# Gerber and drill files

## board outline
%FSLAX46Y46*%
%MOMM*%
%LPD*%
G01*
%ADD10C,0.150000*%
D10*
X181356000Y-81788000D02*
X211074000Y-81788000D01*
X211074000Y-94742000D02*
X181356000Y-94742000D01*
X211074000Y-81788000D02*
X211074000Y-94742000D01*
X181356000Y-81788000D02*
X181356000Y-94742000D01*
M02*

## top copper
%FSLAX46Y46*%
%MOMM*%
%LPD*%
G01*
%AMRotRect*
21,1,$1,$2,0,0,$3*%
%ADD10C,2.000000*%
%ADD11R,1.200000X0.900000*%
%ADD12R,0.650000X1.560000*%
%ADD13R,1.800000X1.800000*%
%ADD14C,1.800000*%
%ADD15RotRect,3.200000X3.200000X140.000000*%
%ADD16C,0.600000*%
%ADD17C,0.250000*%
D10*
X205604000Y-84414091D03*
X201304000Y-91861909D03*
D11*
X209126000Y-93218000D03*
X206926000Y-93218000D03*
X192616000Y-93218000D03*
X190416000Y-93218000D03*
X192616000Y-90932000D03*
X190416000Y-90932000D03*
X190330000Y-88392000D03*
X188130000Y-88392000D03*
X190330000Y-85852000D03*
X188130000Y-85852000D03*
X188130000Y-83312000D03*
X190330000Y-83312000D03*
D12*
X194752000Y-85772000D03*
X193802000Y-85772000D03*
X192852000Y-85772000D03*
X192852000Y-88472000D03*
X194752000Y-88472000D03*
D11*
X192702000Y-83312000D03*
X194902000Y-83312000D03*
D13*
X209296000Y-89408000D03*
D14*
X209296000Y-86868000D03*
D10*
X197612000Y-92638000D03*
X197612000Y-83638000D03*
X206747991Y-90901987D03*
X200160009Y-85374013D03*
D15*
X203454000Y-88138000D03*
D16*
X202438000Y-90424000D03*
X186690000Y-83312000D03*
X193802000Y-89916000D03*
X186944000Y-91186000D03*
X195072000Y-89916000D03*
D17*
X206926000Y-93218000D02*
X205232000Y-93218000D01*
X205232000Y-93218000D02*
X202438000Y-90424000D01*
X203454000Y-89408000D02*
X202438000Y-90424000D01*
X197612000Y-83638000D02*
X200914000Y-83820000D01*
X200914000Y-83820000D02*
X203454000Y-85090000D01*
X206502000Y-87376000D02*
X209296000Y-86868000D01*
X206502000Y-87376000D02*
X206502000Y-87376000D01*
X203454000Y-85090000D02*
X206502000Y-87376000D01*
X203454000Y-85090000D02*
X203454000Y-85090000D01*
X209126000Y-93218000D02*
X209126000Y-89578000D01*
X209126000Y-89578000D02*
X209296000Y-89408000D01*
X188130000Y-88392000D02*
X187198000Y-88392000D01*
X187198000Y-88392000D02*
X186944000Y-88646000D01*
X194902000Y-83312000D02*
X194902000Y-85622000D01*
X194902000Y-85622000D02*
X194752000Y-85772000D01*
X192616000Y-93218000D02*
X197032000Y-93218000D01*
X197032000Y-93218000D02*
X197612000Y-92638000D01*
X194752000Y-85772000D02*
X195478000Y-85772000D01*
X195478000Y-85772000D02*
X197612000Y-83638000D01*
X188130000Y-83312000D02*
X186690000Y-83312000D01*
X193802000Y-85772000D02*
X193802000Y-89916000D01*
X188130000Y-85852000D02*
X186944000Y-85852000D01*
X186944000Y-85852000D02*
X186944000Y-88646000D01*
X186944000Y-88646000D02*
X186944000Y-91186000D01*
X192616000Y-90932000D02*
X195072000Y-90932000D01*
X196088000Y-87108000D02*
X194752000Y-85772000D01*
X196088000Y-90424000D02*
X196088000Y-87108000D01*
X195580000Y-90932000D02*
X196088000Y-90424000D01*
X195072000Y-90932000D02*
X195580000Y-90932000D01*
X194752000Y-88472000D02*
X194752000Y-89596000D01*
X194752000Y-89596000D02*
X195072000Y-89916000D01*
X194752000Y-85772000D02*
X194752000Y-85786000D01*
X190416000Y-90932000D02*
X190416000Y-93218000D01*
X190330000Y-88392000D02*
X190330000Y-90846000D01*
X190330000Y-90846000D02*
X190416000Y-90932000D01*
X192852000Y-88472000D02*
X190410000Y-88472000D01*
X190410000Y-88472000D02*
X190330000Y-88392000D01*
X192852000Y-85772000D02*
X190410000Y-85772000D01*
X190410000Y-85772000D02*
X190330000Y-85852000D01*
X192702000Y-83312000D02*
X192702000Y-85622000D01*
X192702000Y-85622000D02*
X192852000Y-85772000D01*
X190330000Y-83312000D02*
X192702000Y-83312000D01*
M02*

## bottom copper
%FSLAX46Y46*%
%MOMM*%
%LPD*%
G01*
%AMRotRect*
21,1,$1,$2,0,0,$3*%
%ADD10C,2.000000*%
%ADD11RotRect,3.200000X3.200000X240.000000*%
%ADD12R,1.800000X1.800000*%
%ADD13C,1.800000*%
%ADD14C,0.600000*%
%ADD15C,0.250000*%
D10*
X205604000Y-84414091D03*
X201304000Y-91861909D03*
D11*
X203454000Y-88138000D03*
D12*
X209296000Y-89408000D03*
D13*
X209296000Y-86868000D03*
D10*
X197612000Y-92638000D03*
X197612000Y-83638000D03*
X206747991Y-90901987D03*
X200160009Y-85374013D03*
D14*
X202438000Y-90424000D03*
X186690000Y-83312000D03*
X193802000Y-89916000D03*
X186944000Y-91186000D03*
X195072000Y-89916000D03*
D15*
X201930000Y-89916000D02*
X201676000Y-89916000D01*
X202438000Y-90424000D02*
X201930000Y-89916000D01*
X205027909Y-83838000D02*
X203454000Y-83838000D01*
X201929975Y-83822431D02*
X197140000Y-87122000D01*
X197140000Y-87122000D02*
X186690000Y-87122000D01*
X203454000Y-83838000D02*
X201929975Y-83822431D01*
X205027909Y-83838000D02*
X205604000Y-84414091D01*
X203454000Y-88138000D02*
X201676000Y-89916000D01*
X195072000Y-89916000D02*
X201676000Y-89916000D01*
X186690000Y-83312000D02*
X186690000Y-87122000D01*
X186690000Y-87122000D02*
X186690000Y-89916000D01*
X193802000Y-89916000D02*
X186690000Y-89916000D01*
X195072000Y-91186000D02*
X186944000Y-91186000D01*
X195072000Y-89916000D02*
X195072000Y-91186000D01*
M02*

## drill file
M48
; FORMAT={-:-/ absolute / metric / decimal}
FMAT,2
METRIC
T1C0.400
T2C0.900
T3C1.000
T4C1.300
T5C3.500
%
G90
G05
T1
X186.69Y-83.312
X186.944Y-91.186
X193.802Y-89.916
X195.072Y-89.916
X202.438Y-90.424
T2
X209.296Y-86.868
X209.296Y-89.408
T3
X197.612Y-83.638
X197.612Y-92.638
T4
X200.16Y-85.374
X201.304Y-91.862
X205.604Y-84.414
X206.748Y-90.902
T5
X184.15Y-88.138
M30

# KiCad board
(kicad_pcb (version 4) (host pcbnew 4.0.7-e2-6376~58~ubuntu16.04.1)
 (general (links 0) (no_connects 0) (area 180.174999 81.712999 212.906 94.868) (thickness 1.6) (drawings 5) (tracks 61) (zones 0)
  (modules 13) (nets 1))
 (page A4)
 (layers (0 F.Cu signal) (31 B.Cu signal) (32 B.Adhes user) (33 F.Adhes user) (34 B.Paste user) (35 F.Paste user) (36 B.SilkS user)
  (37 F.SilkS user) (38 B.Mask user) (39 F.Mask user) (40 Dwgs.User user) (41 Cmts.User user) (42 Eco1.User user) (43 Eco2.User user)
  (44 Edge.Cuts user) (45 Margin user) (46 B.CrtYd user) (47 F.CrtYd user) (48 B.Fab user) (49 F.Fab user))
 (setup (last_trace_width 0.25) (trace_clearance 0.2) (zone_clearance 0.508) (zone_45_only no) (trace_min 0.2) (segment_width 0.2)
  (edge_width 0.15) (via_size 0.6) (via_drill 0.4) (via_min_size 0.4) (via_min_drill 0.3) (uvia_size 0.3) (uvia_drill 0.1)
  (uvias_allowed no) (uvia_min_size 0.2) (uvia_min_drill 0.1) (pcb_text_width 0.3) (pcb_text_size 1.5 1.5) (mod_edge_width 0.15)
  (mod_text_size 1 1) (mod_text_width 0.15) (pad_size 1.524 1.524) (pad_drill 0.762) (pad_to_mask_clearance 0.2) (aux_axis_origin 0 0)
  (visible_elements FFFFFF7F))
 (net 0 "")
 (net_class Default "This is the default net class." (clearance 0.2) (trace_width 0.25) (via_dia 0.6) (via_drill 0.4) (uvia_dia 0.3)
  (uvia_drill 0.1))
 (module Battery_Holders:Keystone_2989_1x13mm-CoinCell (layer B.Cu) (at 203.454 88.138 240)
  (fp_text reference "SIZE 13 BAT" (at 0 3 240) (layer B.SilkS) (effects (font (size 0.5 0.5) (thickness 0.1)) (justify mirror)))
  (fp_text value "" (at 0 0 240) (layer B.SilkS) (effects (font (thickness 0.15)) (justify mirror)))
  (pad 1 thru_hole circle (at -4.3 0 240) (size 2 2) (drill 1.3) (layers *.Cu *.Mask))
  (pad 1 thru_hole circle (at 4.3 0 240) (size 2 2) (drill 1.3) (layers *.Cu *.Mask))
  (pad 2 smd rect (at 0 0 240) (size 3.2 3.2) (layers B.Cu B.Mask)))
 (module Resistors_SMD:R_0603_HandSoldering (layer F.Cu) (at 208.026 93.218 180)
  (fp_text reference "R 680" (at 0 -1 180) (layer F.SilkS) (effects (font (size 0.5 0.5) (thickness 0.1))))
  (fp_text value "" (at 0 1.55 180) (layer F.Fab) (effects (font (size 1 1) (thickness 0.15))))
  (pad 1 smd rect (at -1.1 0 180) (size 1.2 0.9) (layers F.Cu F.Paste F.Mask))
  (pad 2 smd rect (at 1.1 0 180) (size 1.2 0.9) (layers F.Cu F.Paste F.Mask)))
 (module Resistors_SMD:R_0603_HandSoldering (layer F.Cu) (at 191.516 93.218 180)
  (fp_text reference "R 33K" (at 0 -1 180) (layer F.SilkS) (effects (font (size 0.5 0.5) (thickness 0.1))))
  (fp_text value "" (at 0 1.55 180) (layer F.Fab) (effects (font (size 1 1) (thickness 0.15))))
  (pad 1 smd rect (at -1.1 0 180) (size 1.2 0.9) (layers F.Cu F.Paste F.Mask))
  (pad 2 smd rect (at 1.1 0 180) (size 1.2 0.9) (layers F.Cu F.Paste F.Mask)))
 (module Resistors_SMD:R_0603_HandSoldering (layer F.Cu) (at 191.516 90.932 180)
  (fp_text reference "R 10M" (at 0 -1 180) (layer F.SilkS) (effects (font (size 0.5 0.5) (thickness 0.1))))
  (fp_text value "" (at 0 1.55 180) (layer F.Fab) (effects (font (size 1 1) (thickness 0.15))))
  (pad 1 smd rect (at -1.1 0 180) (size 1.2 0.9) (layers F.Cu F.Paste F.Mask))
  (pad 2 smd rect (at 1.1 0 180) (size 1.2 0.9) (layers F.Cu F.Paste F.Mask)))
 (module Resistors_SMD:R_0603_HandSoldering (layer F.Cu) (at 189.23 88.392 180)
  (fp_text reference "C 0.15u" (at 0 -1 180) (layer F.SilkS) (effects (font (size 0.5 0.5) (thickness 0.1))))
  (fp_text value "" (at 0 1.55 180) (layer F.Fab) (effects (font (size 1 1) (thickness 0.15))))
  (pad 1 smd rect (at -1.1 0 180) (size 1.2 0.9) (layers F.Cu F.Paste F.Mask))
  (pad 2 smd rect (at 1.1 0 180) (size 1.2 0.9) (layers F.Cu F.Paste F.Mask)))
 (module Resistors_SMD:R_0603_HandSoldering (layer F.Cu) (at 189.23 85.852 180)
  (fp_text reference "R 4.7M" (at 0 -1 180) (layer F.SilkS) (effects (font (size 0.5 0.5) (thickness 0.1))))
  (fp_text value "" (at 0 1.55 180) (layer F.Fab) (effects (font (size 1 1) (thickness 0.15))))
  (pad 1 smd rect (at -1.1 0 180) (size 1.2 0.9) (layers F.Cu F.Paste F.Mask))
  (pad 2 smd rect (at 1.1 0 180) (size 1.2 0.9) (layers F.Cu F.Paste F.Mask)))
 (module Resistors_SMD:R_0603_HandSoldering (layer F.Cu) (at 189.23 83.312)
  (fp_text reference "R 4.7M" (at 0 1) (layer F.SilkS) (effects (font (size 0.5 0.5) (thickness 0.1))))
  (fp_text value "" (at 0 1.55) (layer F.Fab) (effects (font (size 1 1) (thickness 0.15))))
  (pad 1 smd rect (at -1.1 0) (size 1.2 0.9) (layers F.Cu F.Paste F.Mask))
  (pad 2 smd rect (at 1.1 0) (size 1.2 0.9) (layers F.Cu F.Paste F.Mask)))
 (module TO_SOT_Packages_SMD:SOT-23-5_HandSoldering (layer F.Cu) (at 193.802 87.122 270)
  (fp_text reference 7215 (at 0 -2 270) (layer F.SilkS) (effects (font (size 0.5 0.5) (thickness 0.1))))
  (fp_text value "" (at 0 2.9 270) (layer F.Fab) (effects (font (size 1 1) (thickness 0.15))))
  (pad 1 smd rect (at -1.35 -0.95 270) (size 1.56 0.65) (layers F.Cu F.Paste F.Mask))
  (pad 2 smd rect (at -1.35 0 270) (size 1.56 0.65) (layers F.Cu F.Paste F.Mask))
  (pad 3 smd rect (at -1.35 0.95 270) (size 1.56 0.65) (layers F.Cu F.Paste F.Mask))
  (pad 4 smd rect (at 1.35 0.95 270) (size 1.56 0.65) (layers F.Cu F.Paste F.Mask))
  (pad 5 smd rect (at 1.35 -0.95 270) (size 1.56 0.65) (layers F.Cu F.Paste F.Mask)))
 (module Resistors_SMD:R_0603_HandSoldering (layer F.Cu) (at 193.802 83.312)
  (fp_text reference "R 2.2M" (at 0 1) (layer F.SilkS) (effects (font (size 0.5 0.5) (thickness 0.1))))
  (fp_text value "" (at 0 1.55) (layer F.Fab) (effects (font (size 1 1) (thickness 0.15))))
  (pad 1 smd rect (at -1.1 0) (size 1.2 0.9) (layers F.Cu F.Paste F.Mask))
  (pad 2 smd rect (at 1.1 0) (size 1.2 0.9) (layers F.Cu F.Paste F.Mask)))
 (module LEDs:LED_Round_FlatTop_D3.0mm (layer F.Cu) (at 209.296 89.408 90)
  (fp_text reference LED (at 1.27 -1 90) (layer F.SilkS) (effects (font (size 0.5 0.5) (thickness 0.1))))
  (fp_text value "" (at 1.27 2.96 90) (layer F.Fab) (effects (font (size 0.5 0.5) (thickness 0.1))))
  (pad 1 thru_hole rect (at 0 0 90) (size 1.8 1.8) (drill 0.9) (layers *.Cu *.Mask))
  (pad 2 thru_hole circle (at 2.54 0 90) (size 1.8 1.8) (drill 0.9) (layers *.Cu *.Mask)))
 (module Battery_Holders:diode (layer F.Cu) (at 197.612 88.138 90)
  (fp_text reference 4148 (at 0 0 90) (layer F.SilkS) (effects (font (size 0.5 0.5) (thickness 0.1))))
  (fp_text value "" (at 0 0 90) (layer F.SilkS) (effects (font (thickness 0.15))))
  (pad 1 thru_hole circle (at -4.5 0 90) (size 2 2) (drill 1) (layers *.Cu *.Mask))
  (pad 2 thru_hole circle (at 4.5 0 90) (size 2 2) (drill 1) (layers *.Cu *.Mask)))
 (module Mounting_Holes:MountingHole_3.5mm (layer F.Cu) (at 184.15 88.138)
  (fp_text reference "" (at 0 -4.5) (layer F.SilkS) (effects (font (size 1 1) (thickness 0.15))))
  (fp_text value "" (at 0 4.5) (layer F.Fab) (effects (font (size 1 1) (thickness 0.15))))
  (pad 1 np_thru_hole circle (at 0 0) (size 3.5 3.5) (drill 3.5) (layers *.Cu *.Mask)))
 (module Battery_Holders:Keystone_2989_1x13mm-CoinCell (layer F.Cu) (at 203.454 88.138 140)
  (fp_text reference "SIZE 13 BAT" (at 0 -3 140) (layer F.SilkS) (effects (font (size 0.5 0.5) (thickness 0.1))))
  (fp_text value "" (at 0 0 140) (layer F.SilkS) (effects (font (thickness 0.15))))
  (pad 1 thru_hole circle (at -4.3 0 140) (size 2 2) (drill 1.3) (layers *.Cu *.Mask))
  (pad 1 thru_hole circle (at 4.3 0 140) (size 2 2) (drill 1.3) (layers *.Cu *.Mask))
  (pad 2 smd rect (at 0 0 140) (size 3.2 3.2) (layers F.Cu F.Mask)))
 (gr_line (start 181.356 81.788) (end 211.074 81.788) (angle 90) (layer Edge.Cuts) (width 0.15))
 (gr_line (start 211.074 94.742) (end 181.356 94.742) (angle 90) (layer Edge.Cuts) (width 0.15))
 (gr_line (start 211.074 81.788) (end 211.074 94.742) (angle 90) (layer Edge.Cuts) (width 0.15))
 (gr_line (start 181.356 81.788) (end 181.356 94.742) (angle 90) (layer Edge.Cuts) (width 0.15))
 (segment (start 206.926 93.218) (end 205.232 93.218) (width 0.25) (layer F.Cu) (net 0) (status 400000))
 (segment (start 205.232 93.218) (end 202.438 90.424) (width 0.25) (layer F.Cu) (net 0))
 (segment (start 203.454 89.408) (end 202.438 90.424) (width 0.25) (layer F.Cu) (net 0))
 (segment (start 201.93 89.916) (end 201.676 89.916) (width 0.25) (layer B.Cu) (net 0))
 (segment (start 202.438 90.424) (end 201.93 89.916) (width 0.25) (layer B.Cu) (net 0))
 (via (at 202.438 90.424) (size 0.6) (drill 0.4) (layers F.Cu B.Cu) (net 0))
 (segment (start 205.027909 83.838) (end 203.454 83.838) (width 0.25) (layer B.Cu) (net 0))
 (segment (start 201.929975 83.822431) (end 197.14 87.122) (width 0.25) (layer B.Cu) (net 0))
 (segment (start 197.14 87.122) (end 186.69 87.122) (width 0.25) (layer B.Cu) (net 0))
 (segment (start 203.454 83.838) (end 201.929975 83.822431) (width 0.25) (layer B.Cu) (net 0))
 (segment (start 205.027909 83.838) (end 205.604 84.414091) (width 0.25) (layer B.Cu) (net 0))
 (segment (start 203.454 88.138) (end 201.676 89.916) (width 0.25) (layer B.Cu) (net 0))
 (segment (start 195.072 89.916) (end 201.676 89.916) (width 0.25) (layer B.Cu) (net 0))
 (segment (start 197.612 83.638) (end 200.914 83.82) (width 0.25) (layer F.Cu) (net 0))
 (segment (start 200.914 83.82) (end 203.454 85.09) (width 0.25) (layer F.Cu) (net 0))
 (segment (start 206.502 87.376) (end 209.296 86.868) (width 0.25) (layer F.Cu) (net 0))
 (segment (start 206.502 87.376) (end 206.502 87.376) (width 0.25) (layer F.Cu) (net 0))
 (segment (start 203.454 85.09) (end 206.502 87.376) (width 0.25) (layer F.Cu) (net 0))
 (segment (start 203.454 85.09) (end 203.454 85.09) (width 0.25) (layer F.Cu) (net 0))
 (segment (start 209.126 93.218) (end 209.126 89.578) (width 0.25) (layer F.Cu) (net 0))
 (segment (start 209.126 89.578) (end 209.296 89.408) (width 0.25) (layer F.Cu) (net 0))
 (segment (start 188.13 88.392) (end 187.198 88.392) (width 0.25) (layer F.Cu) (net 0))
 (segment (start 187.198 88.392) (end 186.944 88.646) (width 0.25) (layer F.Cu) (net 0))
 (segment (start 194.902 83.312) (end 194.902 85.622) (width 0.25) (layer F.Cu) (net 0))
 (segment (start 194.902 85.622) (end 194.752 85.772) (width 0.25) (layer F.Cu) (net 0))
 (segment (start 192.616 93.218) (end 197.032 93.218) (width 0.25) (layer F.Cu) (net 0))
 (segment (start 197.032 93.218) (end 197.612 92.638) (width 0.25) (layer F.Cu) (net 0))
 (segment (start 194.752 85.772) (end 195.478 85.772) (width 0.25) (layer F.Cu) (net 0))
 (segment (start 195.478 85.772) (end 197.612 83.638) (width 0.25) (layer F.Cu) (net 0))
 (segment (start 188.13 83.312) (end 186.69 83.312) (width 0.25) (layer F.Cu) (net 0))
 (via (at 186.69 83.312) (size 0.6) (drill 0.4) (layers F.Cu B.Cu) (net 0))
 (segment (start 186.69 83.312) (end 186.69 87.122) (width 0.25) (layer B.Cu) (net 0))
 (segment (start 186.69 87.122) (end 186.69 89.916) (width 0.25) (layer B.Cu) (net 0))
 (via (at 193.802 89.916) (size 0.6) (drill 0.4) (layers F.Cu B.Cu) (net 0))
 (segment (start 193.802 89.916) (end 186.69 89.916) (width 0.25) (layer B.Cu) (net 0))
 (segment (start 193.802 85.772) (end 193.802 89.916) (width 0.25) (layer F.Cu) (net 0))
 (segment (start 188.13 85.852) (end 186.944 85.852) (width 0.25) (layer F.Cu) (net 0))
 (via (at 186.944 91.186) (size 0.6) (drill 0.4) (layers F.Cu B.Cu) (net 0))
 (segment (start 186.944 85.852) (end 186.944 88.646) (width 0.25) (layer F.Cu) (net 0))
 (segment (start 186.944 88.646) (end 186.944 91.186) (width 0.25) (layer F.Cu) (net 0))
 (segment (start 192.616 90.932) (end 195.072 90.932) (width 0.25) (layer F.Cu) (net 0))
 (segment (start 196.088 87.108) (end 194.752 85.772) (width 0.25) (layer F.Cu) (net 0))
 (segment (start 196.088 90.424) (end 196.088 87.108) (width 0.25) (layer F.Cu) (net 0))
 (segment (start 195.58 90.932) (end 196.088 90.424) (width 0.25) (layer F.Cu) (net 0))
 (segment (start 195.072 90.932) (end 195.58 90.932) (width 0.25) (layer F.Cu) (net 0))
 (segment (start 194.752 88.472) (end 194.752 89.596) (width 0.25) (layer F.Cu) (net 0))
 (segment (start 195.072 91.186) (end 186.944 91.186) (width 0.25) (layer B.Cu) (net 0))
 (segment (start 195.072 89.916) (end 195.072 91.186) (width 0.25) (layer B.Cu) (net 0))
 (via (at 195.072 89.916) (size 0.6) (drill 0.4) (layers F.Cu B.Cu) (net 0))
 (segment (start 194.752 89.596) (end 195.072 89.916) (width 0.25) (layer F.Cu) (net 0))
 (segment (start 194.752 85.772) (end 194.752 85.786) (width 0.25) (layer F.Cu) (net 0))
 (segment (start 190.416 90.932) (end 190.416 93.218) (width 0.25) (layer F.Cu) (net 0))
 (segment (start 190.33 88.392) (end 190.33 90.846) (width 0.25) (layer F.Cu) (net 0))
 (segment (start 190.33 90.846) (end 190.416 90.932) (width 0.25) (layer F.Cu) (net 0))
 (segment (start 192.852 88.472) (end 190.41 88.472) (width 0.25) (layer F.Cu) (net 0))
 (segment (start 190.41 88.472) (end 190.33 88.392) (width 0.25) (layer F.Cu) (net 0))
 (segment (start 192.852 85.772) (end 190.41 85.772) (width 0.25) (layer F.Cu) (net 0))
 (segment (start 190.41 85.772) (end 190.33 85.852) (width 0.25) (layer F.Cu) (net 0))
 (segment (start 192.702 83.312) (end 192.702 85.622) (width 0.25) (layer F.Cu) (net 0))
 (segment (start 192.702 85.622) (end 192.852 85.772) (width 0.25) (layer F.Cu) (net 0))
 (segment (start 190.33 83.312) (end 192.702 83.312) (width 0.25) (layer F.Cu) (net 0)))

